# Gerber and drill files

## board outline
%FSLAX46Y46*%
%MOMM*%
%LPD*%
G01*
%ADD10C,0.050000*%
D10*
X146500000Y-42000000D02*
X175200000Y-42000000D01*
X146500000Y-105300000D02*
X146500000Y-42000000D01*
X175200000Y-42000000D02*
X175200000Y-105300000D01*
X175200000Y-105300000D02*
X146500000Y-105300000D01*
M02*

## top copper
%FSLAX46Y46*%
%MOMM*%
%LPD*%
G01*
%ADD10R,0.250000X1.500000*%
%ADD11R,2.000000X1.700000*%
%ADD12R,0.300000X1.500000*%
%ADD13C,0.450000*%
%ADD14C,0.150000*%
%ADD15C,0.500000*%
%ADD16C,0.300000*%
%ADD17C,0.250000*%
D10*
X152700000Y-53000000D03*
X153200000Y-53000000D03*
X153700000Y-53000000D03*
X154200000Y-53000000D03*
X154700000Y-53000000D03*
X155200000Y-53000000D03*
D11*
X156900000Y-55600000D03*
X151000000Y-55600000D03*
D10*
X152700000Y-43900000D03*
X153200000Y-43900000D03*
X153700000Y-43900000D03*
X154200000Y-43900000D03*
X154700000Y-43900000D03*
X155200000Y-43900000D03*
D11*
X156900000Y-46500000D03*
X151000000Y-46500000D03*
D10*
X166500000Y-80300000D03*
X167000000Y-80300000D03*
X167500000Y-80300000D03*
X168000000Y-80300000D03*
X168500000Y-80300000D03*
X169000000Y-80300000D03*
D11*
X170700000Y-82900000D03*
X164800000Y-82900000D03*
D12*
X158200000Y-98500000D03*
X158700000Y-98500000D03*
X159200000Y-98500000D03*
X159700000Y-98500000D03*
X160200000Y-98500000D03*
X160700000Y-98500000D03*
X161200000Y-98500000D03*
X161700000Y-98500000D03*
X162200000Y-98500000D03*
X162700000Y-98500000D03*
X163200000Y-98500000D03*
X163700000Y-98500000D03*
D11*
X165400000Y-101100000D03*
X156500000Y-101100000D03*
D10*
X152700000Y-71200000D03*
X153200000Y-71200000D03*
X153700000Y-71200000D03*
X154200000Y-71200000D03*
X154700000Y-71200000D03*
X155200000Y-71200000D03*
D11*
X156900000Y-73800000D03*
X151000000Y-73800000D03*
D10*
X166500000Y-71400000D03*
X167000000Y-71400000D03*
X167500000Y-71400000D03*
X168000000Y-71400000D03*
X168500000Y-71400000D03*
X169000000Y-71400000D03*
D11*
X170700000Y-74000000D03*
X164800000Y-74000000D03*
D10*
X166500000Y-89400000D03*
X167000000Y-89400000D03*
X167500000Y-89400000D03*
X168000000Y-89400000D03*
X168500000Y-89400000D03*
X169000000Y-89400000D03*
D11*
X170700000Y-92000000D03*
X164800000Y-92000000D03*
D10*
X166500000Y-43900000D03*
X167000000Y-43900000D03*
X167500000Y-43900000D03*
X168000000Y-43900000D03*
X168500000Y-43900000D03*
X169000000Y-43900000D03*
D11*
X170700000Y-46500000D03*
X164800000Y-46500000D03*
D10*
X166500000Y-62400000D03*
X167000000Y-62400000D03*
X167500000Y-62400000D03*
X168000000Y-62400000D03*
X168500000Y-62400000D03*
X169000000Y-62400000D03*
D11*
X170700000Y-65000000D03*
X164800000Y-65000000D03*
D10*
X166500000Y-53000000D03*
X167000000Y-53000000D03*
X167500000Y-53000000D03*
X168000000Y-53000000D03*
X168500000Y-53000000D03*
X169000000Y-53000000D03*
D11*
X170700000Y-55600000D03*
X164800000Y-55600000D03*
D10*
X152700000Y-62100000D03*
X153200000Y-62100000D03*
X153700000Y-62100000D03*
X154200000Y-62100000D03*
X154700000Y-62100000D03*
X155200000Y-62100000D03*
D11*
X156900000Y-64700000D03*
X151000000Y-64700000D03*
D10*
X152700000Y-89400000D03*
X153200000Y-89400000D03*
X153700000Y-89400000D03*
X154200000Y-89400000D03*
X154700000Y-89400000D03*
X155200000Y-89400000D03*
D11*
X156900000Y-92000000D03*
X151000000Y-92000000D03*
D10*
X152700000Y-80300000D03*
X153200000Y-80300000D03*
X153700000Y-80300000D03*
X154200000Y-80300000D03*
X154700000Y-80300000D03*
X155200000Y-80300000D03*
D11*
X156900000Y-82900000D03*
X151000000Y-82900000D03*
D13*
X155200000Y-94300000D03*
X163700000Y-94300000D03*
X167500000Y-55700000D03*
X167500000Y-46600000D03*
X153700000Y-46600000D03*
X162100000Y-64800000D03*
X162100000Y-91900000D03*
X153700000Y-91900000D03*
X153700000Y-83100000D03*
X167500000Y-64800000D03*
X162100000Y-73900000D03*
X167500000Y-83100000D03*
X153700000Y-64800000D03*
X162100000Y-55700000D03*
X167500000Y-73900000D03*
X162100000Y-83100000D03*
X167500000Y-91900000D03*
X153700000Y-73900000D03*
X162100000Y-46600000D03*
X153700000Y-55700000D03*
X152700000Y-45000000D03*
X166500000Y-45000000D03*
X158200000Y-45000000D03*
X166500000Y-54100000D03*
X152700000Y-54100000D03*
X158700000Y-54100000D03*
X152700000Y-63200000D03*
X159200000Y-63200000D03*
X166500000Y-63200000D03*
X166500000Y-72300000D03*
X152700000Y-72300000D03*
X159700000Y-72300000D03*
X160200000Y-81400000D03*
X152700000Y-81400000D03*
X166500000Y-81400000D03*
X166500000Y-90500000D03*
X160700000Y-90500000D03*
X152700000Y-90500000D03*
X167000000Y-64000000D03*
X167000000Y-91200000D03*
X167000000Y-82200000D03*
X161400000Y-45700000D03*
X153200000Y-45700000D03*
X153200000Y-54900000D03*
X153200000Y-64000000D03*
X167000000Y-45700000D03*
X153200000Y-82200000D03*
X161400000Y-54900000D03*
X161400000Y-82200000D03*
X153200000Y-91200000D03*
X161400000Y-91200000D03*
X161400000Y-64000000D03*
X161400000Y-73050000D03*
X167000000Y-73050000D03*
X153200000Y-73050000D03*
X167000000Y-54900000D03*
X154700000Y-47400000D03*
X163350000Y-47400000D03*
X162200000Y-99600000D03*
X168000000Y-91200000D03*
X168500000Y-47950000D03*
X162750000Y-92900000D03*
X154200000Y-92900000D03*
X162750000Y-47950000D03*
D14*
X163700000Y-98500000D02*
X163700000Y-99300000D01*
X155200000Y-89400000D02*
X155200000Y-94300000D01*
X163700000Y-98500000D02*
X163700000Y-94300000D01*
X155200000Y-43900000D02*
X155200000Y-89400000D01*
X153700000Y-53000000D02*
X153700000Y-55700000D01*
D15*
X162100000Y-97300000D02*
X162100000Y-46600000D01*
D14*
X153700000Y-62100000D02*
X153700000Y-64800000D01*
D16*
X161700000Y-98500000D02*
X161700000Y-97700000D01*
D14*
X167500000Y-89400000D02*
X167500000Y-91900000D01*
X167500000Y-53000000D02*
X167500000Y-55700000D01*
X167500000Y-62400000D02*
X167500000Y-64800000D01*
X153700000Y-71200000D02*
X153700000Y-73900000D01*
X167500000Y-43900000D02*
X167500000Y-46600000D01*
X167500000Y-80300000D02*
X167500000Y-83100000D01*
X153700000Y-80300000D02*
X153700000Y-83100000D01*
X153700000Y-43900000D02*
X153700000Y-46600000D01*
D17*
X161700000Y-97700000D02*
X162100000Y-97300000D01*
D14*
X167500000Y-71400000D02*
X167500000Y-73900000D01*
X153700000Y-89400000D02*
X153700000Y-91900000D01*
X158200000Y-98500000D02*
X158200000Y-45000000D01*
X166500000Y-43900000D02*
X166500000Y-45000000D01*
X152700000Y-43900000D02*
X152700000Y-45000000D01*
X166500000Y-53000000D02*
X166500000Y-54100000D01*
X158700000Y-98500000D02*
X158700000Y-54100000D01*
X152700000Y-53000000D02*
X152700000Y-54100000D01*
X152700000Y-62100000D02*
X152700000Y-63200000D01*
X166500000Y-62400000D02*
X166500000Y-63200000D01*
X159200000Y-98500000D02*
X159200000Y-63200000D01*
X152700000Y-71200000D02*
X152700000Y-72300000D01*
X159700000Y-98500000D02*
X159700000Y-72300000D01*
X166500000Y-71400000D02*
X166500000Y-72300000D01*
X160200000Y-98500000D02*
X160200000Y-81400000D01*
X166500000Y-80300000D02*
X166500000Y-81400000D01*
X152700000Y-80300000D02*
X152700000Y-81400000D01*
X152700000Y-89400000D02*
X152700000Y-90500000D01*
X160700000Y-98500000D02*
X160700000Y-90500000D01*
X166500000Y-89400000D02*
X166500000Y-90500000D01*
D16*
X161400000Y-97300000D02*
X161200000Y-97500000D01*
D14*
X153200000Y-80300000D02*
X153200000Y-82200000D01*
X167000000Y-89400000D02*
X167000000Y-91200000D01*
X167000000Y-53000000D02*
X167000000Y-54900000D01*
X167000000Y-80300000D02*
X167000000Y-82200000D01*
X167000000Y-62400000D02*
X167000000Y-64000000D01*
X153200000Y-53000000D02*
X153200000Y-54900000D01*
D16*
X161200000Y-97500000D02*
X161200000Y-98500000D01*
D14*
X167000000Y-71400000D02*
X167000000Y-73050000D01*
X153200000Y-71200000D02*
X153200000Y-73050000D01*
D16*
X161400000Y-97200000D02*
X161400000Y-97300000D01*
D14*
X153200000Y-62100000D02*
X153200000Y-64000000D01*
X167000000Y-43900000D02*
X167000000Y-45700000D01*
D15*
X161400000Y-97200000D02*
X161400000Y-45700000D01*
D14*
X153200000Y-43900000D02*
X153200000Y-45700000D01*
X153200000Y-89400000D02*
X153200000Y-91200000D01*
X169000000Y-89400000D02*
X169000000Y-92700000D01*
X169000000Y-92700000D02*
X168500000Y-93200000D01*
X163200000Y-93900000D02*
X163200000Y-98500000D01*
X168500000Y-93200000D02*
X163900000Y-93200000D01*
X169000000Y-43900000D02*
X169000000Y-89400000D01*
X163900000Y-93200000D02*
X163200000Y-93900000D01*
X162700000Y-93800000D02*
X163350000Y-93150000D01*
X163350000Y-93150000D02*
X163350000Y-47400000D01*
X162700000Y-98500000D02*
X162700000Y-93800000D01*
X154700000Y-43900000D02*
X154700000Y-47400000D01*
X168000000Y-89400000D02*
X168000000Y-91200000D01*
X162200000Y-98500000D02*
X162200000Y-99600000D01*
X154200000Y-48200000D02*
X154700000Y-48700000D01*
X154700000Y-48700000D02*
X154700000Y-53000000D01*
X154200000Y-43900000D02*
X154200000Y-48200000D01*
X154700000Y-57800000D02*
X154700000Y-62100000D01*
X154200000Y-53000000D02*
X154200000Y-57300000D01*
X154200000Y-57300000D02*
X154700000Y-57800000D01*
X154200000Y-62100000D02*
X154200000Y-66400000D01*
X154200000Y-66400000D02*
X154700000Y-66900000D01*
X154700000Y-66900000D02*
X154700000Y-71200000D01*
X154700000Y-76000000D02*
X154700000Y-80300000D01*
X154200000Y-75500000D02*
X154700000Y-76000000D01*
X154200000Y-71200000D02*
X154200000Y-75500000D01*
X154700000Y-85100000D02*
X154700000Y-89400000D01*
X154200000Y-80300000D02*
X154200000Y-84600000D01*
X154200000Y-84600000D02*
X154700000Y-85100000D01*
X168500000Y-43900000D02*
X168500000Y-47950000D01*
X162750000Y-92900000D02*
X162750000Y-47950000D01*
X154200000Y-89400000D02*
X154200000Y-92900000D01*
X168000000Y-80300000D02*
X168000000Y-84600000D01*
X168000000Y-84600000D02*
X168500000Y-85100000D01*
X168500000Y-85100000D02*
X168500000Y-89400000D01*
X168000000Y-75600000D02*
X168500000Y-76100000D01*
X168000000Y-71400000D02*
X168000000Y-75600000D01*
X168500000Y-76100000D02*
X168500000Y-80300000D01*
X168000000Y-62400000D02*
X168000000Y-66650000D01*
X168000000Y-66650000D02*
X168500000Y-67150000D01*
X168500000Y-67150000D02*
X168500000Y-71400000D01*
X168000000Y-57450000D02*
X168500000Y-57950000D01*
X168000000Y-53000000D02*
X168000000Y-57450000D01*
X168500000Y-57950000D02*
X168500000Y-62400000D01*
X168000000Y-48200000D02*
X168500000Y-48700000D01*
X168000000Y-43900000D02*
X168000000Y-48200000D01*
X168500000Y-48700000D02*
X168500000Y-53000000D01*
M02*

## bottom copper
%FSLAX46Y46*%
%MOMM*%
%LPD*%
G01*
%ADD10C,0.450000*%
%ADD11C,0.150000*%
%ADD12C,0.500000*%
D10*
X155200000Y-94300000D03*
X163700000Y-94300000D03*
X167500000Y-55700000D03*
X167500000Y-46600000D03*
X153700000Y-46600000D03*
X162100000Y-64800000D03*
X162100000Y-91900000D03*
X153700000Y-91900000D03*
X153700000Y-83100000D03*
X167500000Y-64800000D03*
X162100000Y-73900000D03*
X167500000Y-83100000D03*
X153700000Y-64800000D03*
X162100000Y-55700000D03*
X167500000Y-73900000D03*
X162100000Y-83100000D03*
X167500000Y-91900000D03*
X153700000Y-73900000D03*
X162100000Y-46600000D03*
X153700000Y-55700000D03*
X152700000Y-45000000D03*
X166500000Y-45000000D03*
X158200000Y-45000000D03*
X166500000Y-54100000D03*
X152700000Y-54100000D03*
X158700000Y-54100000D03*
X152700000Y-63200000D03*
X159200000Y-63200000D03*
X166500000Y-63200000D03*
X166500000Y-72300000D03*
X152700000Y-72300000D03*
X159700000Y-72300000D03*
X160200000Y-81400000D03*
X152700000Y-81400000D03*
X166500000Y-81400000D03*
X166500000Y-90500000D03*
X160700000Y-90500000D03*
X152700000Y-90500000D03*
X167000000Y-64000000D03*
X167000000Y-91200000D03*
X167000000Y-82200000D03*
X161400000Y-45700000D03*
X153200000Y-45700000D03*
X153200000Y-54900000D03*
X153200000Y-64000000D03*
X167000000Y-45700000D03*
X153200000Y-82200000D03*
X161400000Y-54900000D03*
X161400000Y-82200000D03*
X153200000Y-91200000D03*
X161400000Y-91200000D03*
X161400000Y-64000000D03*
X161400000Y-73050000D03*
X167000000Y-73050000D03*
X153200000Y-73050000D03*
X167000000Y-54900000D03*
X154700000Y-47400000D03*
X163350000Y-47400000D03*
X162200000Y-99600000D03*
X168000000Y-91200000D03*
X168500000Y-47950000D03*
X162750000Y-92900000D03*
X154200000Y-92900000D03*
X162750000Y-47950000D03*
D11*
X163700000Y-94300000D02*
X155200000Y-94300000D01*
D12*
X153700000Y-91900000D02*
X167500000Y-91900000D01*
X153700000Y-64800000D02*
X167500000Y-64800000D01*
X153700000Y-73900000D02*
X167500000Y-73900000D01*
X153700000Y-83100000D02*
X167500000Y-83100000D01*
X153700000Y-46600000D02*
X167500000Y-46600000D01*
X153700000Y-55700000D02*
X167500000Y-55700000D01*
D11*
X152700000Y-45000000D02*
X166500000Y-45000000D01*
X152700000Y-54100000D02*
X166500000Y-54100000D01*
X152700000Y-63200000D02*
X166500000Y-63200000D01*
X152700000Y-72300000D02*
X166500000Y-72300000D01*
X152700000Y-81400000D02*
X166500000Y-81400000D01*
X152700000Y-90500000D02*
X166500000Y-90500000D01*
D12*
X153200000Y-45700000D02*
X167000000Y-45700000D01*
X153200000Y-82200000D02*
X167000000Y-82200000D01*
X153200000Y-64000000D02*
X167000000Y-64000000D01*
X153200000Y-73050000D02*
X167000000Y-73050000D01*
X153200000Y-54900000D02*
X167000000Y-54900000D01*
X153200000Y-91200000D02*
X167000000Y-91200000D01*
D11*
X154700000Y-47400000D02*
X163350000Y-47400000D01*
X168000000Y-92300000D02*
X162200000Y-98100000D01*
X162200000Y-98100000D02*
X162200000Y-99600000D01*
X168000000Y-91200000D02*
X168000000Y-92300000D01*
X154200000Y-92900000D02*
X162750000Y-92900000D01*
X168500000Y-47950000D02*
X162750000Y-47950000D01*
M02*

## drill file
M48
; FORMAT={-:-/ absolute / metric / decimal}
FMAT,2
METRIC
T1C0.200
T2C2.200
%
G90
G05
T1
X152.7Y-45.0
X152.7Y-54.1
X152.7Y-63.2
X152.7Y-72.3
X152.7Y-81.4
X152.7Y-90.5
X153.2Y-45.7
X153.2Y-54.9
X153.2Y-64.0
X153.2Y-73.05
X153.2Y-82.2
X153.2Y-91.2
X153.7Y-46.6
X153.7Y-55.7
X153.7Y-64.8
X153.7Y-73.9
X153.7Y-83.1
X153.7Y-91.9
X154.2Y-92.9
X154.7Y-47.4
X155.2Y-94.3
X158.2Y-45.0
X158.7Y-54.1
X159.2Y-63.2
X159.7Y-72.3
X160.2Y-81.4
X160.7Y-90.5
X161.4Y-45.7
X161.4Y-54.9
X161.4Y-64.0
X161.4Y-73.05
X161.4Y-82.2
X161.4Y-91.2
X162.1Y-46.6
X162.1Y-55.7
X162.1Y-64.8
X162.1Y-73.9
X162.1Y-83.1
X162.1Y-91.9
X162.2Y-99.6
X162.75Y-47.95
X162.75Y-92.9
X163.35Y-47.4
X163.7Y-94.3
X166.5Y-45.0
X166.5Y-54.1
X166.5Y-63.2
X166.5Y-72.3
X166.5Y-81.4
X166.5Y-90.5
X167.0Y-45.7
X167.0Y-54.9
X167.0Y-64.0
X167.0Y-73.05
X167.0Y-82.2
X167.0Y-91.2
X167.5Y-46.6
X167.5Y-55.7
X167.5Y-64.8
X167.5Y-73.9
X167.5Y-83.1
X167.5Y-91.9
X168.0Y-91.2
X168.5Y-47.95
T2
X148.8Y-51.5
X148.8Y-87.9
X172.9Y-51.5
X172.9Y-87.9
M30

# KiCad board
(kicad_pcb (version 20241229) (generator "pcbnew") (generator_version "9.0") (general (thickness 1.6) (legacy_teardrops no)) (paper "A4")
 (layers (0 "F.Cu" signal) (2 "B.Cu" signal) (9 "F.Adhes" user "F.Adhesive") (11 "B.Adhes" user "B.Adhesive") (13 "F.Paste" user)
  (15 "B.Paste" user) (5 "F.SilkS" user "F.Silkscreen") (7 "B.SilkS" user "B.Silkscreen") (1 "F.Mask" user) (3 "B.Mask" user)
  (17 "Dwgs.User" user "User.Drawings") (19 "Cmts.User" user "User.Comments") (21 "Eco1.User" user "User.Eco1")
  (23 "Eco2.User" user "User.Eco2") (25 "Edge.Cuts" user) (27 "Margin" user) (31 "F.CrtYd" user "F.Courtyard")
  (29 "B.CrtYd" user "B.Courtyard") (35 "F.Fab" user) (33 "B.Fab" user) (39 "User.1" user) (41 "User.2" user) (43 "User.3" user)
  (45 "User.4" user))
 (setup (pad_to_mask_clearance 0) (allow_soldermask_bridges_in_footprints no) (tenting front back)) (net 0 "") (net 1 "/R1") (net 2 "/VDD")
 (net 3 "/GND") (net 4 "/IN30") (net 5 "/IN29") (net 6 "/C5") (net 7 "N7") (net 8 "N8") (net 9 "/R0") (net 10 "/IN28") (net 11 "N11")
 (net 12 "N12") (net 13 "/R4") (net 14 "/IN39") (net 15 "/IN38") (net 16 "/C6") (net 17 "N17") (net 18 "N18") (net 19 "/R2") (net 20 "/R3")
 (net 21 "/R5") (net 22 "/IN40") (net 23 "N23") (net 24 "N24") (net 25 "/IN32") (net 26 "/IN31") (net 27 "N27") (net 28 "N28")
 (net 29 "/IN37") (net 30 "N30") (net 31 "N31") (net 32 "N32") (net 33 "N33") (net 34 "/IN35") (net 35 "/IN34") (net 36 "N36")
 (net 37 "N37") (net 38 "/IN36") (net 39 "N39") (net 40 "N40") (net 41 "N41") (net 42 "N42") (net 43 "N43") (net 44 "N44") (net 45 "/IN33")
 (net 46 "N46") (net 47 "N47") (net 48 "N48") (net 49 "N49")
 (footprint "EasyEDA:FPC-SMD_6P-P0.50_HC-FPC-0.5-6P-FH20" (layer "F.Cu") (at 153.95 54.3)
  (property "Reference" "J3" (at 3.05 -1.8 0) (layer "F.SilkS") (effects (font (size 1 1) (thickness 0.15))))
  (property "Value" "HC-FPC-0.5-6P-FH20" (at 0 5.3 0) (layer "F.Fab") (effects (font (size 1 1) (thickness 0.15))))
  (pad "1" smd rect (at -1.25 -1.3) (size 0.25 1.5) (layers "F.Cu" "F.Mask" "F.Paste") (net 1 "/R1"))
  (pad "2" smd rect (at -0.75 -1.3) (size 0.25 1.5) (layers "F.Cu" "F.Mask" "F.Paste") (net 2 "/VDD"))
  (pad "3" smd rect (at -0.25 -1.3) (size 0.25 1.5) (layers "F.Cu" "F.Mask" "F.Paste") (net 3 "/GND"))
  (pad "4" smd rect (at 0.25 -1.3) (size 0.25 1.5) (layers "F.Cu" "F.Mask" "F.Paste") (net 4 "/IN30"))
  (pad "5" smd rect (at 0.75 -1.3) (size 0.25 1.5) (layers "F.Cu" "F.Mask" "F.Paste") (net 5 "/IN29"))
  (pad "6" smd rect (at 1.25 -1.3) (size 0.25 1.5) (layers "F.Cu" "F.Mask" "F.Paste") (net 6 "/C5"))
  (pad "7" smd rect (at 2.95 1.3) (size 2 1.7) (layers "F.Cu" "F.Mask" "F.Paste") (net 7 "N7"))
  (pad "8" smd rect (at -2.95 1.3) (size 2 1.7) (layers "F.Cu" "F.Mask" "F.Paste") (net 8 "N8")))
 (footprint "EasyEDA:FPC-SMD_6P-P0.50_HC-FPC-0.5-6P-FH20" (layer "F.Cu") (at 153.95 45.2)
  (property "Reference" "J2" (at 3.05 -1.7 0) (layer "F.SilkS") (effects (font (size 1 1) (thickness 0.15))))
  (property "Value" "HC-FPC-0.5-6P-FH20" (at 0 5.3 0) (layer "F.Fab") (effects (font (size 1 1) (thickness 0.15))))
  (pad "1" smd rect (at -1.25 -1.3) (size 0.25 1.5) (layers "F.Cu" "F.Mask" "F.Paste") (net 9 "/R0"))
  (pad "2" smd rect (at -0.75 -1.3) (size 0.25 1.5) (layers "F.Cu" "F.Mask" "F.Paste") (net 2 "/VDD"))
  (pad "3" smd rect (at -0.25 -1.3) (size 0.25 1.5) (layers "F.Cu" "F.Mask" "F.Paste") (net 3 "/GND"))
  (pad "4" smd rect (at 0.25 -1.3) (size 0.25 1.5) (layers "F.Cu" "F.Mask" "F.Paste") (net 5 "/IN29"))
  (pad "5" smd rect (at 0.75 -1.3) (size 0.25 1.5) (layers "F.Cu" "F.Mask" "F.Paste") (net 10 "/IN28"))
  (pad "6" smd rect (at 1.25 -1.3) (size 0.25 1.5) (layers "F.Cu" "F.Mask" "F.Paste") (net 6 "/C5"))
  (pad "7" smd rect (at 2.95 1.3) (size 2 1.7) (layers "F.Cu" "F.Mask" "F.Paste") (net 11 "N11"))
  (pad "8" smd rect (at -2.95 1.3) (size 2 1.7) (layers "F.Cu" "F.Mask" "F.Paste") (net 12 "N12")))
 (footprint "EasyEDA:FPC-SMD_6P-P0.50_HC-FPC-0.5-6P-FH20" (layer "F.Cu") (at 167.75 81.6)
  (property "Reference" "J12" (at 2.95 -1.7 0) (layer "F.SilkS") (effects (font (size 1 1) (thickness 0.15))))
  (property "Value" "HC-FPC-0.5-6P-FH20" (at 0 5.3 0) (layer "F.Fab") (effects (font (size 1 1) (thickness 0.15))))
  (pad "1" smd rect (at -1.25 -1.3) (size 0.25 1.5) (layers "F.Cu" "F.Mask" "F.Paste") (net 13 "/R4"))
  (pad "2" smd rect (at -0.75 -1.3) (size 0.25 1.5) (layers "F.Cu" "F.Mask" "F.Paste") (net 2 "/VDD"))
  (pad "3" smd rect (at -0.25 -1.3) (size 0.25 1.5) (layers "F.Cu" "F.Mask" "F.Paste") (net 3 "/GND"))
  (pad "4" smd rect (at 0.25 -1.3) (size 0.25 1.5) (layers "F.Cu" "F.Mask" "F.Paste") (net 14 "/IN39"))
  (pad "5" smd rect (at 0.75 -1.3) (size 0.25 1.5) (layers "F.Cu" "F.Mask" "F.Paste") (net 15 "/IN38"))
  (pad "6" smd rect (at 1.25 -1.3) (size 0.25 1.5) (layers "F.Cu" "F.Mask" "F.Paste") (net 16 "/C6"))
  (pad "7" smd rect (at 2.95 1.3) (size 2 1.7) (layers "F.Cu" "F.Mask" "F.Paste") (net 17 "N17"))
  (pad "8" smd rect (at -2.95 1.3) (size 2 1.7) (layers "F.Cu" "F.Mask" "F.Paste") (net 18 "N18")))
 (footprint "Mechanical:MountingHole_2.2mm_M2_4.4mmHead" (layer "F.Cu") (at 148.8 87.9)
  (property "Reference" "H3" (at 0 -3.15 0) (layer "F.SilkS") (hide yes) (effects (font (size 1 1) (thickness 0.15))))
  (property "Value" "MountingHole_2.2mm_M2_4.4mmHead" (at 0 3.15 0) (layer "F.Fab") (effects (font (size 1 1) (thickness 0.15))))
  (pad "" np_thru_hole circle (at 0 0) (size 2.2 2.2) (drill 2.2) (layers "*.Cu" "*.Mask")))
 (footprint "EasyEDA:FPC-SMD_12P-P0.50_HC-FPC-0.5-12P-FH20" (layer "F.Cu") (at 160.95 99.8)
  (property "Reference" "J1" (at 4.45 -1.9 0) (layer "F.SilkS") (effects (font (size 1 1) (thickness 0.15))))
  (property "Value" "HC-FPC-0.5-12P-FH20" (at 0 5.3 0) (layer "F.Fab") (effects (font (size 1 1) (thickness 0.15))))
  (pad "1" smd rect (at -2.75 -1.3) (size 0.3 1.5) (layers "F.Cu" "F.Mask" "F.Paste") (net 9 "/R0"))
  (pad "2" smd rect (at -2.25 -1.3) (size 0.3 1.5) (layers "F.Cu" "F.Mask" "F.Paste") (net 1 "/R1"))
  (pad "3" smd rect (at -1.75 -1.3) (size 0.3 1.5) (layers "F.Cu" "F.Mask" "F.Paste") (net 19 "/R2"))
  (pad "4" smd rect (at -1.25 -1.3) (size 0.3 1.5) (layers "F.Cu" "F.Mask" "F.Paste") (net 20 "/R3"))
  (pad "5" smd rect (at -0.75 -1.3) (size 0.3 1.5) (layers "F.Cu" "F.Mask" "F.Paste") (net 13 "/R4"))
  (pad "6" smd rect (at -0.25 -1.3) (size 0.3 1.5) (layers "F.Cu" "F.Mask" "F.Paste") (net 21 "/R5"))
  (pad "7" smd rect (at 0.25 -1.3) (size 0.3 1.5) (layers "F.Cu" "F.Mask" "F.Paste") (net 2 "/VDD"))
  (pad "8" smd rect (at 0.75 -1.3) (size 0.3 1.5) (layers "F.Cu" "F.Mask" "F.Paste") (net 3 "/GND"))
  (pad "9" smd rect (at 1.25 -1.3) (size 0.3 1.5) (layers "F.Cu" "F.Mask" "F.Paste") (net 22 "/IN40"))
  (pad "10" smd rect (at 1.75 -1.3) (size 0.3 1.5) (layers "F.Cu" "F.Mask" "F.Paste") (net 10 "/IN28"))
  (pad "11" smd rect (at 2.25 -1.3) (size 0.3 1.5) (layers "F.Cu" "F.Mask" "F.Paste") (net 16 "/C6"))
  (pad "12" smd rect (at 2.75 -1.3) (size 0.3 1.5) (layers "F.Cu" "F.Mask" "F.Paste") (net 6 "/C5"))
  (pad "13" smd rect (at 4.45 1.3) (size 2 1.7) (layers "F.Cu" "F.Mask" "F.Paste") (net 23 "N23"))
  (pad "14" smd rect (at -4.45 1.3) (size 2 1.7) (layers "F.Cu" "F.Mask" "F.Paste") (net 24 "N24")))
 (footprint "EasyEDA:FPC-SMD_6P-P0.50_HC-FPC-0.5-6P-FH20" (layer "F.Cu") (at 153.95 72.5)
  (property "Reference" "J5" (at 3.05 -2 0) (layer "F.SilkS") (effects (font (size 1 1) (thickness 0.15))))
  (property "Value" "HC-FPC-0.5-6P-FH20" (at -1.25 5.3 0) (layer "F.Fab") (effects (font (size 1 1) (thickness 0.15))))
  (pad "1" smd rect (at -1.25 -1.3) (size 0.25 1.5) (layers "F.Cu" "F.Mask" "F.Paste") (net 20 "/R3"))
  (pad "2" smd rect (at -0.75 -1.3) (size 0.25 1.5) (layers "F.Cu" "F.Mask" "F.Paste") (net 2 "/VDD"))
  (pad "3" smd rect (at -0.25 -1.3) (size 0.25 1.5) (layers "F.Cu" "F.Mask" "F.Paste") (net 3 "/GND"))
  (pad "4" smd rect (at 0.25 -1.3) (size 0.25 1.5) (layers "F.Cu" "F.Mask" "F.Paste") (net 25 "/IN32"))
  (pad "5" smd rect (at 0.75 -1.3) (size 0.25 1.5) (layers "F.Cu" "F.Mask" "F.Paste") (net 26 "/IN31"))
  (pad "6" smd rect (at 1.25 -1.3) (size 0.25 1.5) (layers "F.Cu" "F.Mask" "F.Paste") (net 6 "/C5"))
  (pad "7" smd rect (at 2.95 1.3) (size 2 1.7) (layers "F.Cu" "F.Mask" "F.Paste") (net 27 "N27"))
  (pad "8" smd rect (at -2.95 1.3) (size 2 1.7) (layers "F.Cu" "F.Mask" "F.Paste") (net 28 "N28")))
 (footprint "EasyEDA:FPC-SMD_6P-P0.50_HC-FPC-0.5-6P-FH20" (layer "F.Cu") (at 167.75 72.7)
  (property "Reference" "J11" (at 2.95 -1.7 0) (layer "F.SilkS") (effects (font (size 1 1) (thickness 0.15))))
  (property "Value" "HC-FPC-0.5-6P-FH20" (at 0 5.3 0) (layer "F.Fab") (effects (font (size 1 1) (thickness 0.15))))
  (pad "1" smd rect (at -1.25 -1.3) (size 0.25 1.5) (layers "F.Cu" "F.Mask" "F.Paste") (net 20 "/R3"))
  (pad "2" smd rect (at -0.75 -1.3) (size 0.25 1.5) (layers "F.Cu" "F.Mask" "F.Paste") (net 2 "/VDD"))
  (pad "3" smd rect (at -0.25 -1.3) (size 0.25 1.5) (layers "F.Cu" "F.Mask" "F.Paste") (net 3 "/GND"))
  (pad "4" smd rect (at 0.25 -1.3) (size 0.25 1.5) (layers "F.Cu" "F.Mask" "F.Paste") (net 15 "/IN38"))
  (pad "5" smd rect (at 0.75 -1.3) (size 0.25 1.5) (layers "F.Cu" "F.Mask" "F.Paste") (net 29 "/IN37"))
  (pad "6" smd rect (at 1.25 -1.3) (size 0.25 1.5) (layers "F.Cu" "F.Mask" "F.Paste") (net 16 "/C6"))
  (pad "7" smd rect (at 2.95 1.3) (size 2 1.7) (layers "F.Cu" "F.Mask" "F.Paste") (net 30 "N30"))
  (pad "8" smd rect (at -2.95 1.3) (size 2 1.7) (layers "F.Cu" "F.Mask" "F.Paste") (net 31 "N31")))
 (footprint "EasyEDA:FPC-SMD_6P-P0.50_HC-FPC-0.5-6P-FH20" (layer "F.Cu") (at 167.75 90.7)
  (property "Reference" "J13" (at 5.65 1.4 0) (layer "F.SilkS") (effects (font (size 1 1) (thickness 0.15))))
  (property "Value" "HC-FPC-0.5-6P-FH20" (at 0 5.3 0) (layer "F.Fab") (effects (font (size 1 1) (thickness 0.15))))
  (pad "1" smd rect (at -1.25 -1.3) (size 0.25 1.5) (layers "F.Cu" "F.Mask" "F.Paste") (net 21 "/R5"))
  (pad "2" smd rect (at -0.75 -1.3) (size 0.25 1.5) (layers "F.Cu" "F.Mask" "F.Paste") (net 2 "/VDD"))
  (pad "3" smd rect (at -0.25 -1.3) (size 0.25 1.5) (layers "F.Cu" "F.Mask" "F.Paste") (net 3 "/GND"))
  (pad "4" smd rect (at 0.25 -1.3) (size 0.25 1.5) (layers "F.Cu" "F.Mask" "F.Paste") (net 22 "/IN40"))
  (pad "5" smd rect (at 0.75 -1.3) (size 0.25 1.5) (layers "F.Cu" "F.Mask" "F.Paste") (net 14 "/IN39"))
  (pad "6" smd rect (at 1.25 -1.3) (size 0.25 1.5) (layers "F.Cu" "F.Mask" "F.Paste") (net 16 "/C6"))
  (pad "7" smd rect (at 2.95 1.3) (size 2 1.7) (layers "F.Cu" "F.Mask" "F.Paste") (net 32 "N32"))
  (pad "8" smd rect (at -2.95 1.3) (size 2 1.7) (layers "F.Cu" "F.Mask" "F.Paste") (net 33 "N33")))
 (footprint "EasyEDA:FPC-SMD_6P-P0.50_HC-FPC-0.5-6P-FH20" (layer "F.Cu") (at 167.75 45.2)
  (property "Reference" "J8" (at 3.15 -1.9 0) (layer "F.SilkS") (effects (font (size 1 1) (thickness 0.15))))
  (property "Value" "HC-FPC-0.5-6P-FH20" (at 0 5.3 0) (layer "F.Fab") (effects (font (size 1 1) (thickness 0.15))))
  (pad "1" smd rect (at -1.25 -1.3) (size 0.25 1.5) (layers "F.Cu" "F.Mask" "F.Paste") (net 9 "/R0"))
  (pad "2" smd rect (at -0.75 -1.3) (size 0.25 1.5) (layers "F.Cu" "F.Mask" "F.Paste") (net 2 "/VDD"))
  (pad "3" smd rect (at -0.25 -1.3) (size 0.25 1.5) (layers "F.Cu" "F.Mask" "F.Paste") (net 3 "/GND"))
  (pad "4" smd rect (at 0.25 -1.3) (size 0.25 1.5) (layers "F.Cu" "F.Mask" "F.Paste") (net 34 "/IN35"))
  (pad "5" smd rect (at 0.75 -1.3) (size 0.25 1.5) (layers "F.Cu" "F.Mask" "F.Paste") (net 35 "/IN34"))
  (pad "6" smd rect (at 1.25 -1.3) (size 0.25 1.5) (layers "F.Cu" "F.Mask" "F.Paste") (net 16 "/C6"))
  (pad "7" smd rect (at 2.95 1.3) (size 2 1.7) (layers "F.Cu" "F.Mask" "F.Paste") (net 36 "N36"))
  (pad "8" smd rect (at -2.95 1.3) (size 2 1.7) (layers "F.Cu" "F.Mask" "F.Paste") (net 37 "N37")))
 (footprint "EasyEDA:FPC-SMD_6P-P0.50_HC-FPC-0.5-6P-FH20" (layer "F.Cu") (at 167.75 63.7)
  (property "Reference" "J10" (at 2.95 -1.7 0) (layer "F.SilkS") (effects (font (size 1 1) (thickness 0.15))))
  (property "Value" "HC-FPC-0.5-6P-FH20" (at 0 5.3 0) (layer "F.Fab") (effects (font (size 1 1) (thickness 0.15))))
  (pad "1" smd rect (at -1.25 -1.3) (size 0.25 1.5) (layers "F.Cu" "F.Mask" "F.Paste") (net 19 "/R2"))
  (pad "2" smd rect (at -0.75 -1.3) (size 0.25 1.5) (layers "F.Cu" "F.Mask" "F.Paste") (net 2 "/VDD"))
  (pad "3" smd rect (at -0.25 -1.3) (size 0.25 1.5) (layers "F.Cu" "F.Mask" "F.Paste") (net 3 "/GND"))
  (pad "4" smd rect (at 0.25 -1.3) (size 0.25 1.5) (layers "F.Cu" "F.Mask" "F.Paste") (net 29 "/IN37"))
  (pad "5" smd rect (at 0.75 -1.3) (size 0.25 1.5) (layers "F.Cu" "F.Mask" "F.Paste") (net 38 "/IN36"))
  (pad "6" smd rect (at 1.25 -1.3) (size 0.25 1.5) (layers "F.Cu" "F.Mask" "F.Paste") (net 16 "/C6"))
  (pad "7" smd rect (at 2.95 1.3) (size 2 1.7) (layers "F.Cu" "F.Mask" "F.Paste") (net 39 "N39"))
  (pad "8" smd rect (at -2.95 1.3) (size 2 1.7) (layers "F.Cu" "F.Mask" "F.Paste") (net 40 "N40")))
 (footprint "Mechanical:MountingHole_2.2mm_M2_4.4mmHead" (layer "F.Cu") (at 172.9 51.5)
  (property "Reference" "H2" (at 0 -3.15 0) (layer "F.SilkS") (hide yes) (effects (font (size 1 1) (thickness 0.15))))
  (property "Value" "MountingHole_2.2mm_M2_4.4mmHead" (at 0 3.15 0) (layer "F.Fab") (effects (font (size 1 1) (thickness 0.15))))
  (pad "" np_thru_hole circle (at 0 0) (size 2.2 2.2) (drill 2.2) (layers "*.Cu" "*.Mask")))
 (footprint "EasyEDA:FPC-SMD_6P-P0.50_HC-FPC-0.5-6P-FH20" (layer "F.Cu") (at 167.75 54.3)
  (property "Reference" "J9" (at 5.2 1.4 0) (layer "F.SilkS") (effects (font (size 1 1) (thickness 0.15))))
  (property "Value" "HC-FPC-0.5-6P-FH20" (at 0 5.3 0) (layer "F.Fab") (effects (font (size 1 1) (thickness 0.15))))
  (pad "1" smd rect (at -1.25 -1.3) (size 0.25 1.5) (layers "F.Cu" "F.Mask" "F.Paste") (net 1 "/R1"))
  (pad "2" smd rect (at -0.75 -1.3) (size 0.25 1.5) (layers "F.Cu" "F.Mask" "F.Paste") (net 2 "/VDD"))
  (pad "3" smd rect (at -0.25 -1.3) (size 0.25 1.5) (layers "F.Cu" "F.Mask" "F.Paste") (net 3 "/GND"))
  (pad "4" smd rect (at 0.25 -1.3) (size 0.25 1.5) (layers "F.Cu" "F.Mask" "F.Paste") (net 38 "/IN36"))
  (pad "5" smd rect (at 0.75 -1.3) (size 0.25 1.5) (layers "F.Cu" "F.Mask" "F.Paste") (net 34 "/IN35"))
  (pad "6" smd rect (at 1.25 -1.3) (size 0.25 1.5) (layers "F.Cu" "F.Mask" "F.Paste") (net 16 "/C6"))
  (pad "7" smd rect (at 2.95 1.3) (size 2 1.7) (layers "F.Cu" "F.Mask" "F.Paste") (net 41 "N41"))
  (pad "8" smd rect (at -2.95 1.3) (size 2 1.7) (layers "F.Cu" "F.Mask" "F.Paste") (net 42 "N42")))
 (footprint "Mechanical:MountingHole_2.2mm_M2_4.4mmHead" (layer "F.Cu") (at 148.8 51.5)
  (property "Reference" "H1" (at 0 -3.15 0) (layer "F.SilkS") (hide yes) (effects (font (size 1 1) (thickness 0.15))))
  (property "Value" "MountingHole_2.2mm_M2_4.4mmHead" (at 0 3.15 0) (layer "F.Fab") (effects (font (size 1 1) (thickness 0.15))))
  (pad "" np_thru_hole circle (at 0 0) (size 2.2 2.2) (drill 2.2) (layers "*.Cu" "*.Mask")))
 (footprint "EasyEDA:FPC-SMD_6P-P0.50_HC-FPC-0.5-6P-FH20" (layer "F.Cu") (at 153.95 63.4)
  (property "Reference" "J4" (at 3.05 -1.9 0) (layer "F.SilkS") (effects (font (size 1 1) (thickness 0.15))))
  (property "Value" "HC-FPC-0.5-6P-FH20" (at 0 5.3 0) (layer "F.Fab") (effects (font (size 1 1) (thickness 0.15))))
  (pad "1" smd rect (at -1.25 -1.3) (size 0.25 1.5) (layers "F.Cu" "F.Mask" "F.Paste") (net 19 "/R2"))
  (pad "2" smd rect (at -0.75 -1.3) (size 0.25 1.5) (layers "F.Cu" "F.Mask" "F.Paste") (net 2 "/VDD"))
  (pad "3" smd rect (at -0.25 -1.3) (size 0.25 1.5) (layers "F.Cu" "F.Mask" "F.Paste") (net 3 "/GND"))
  (pad "4" smd rect (at 0.25 -1.3) (size 0.25 1.5) (layers "F.Cu" "F.Mask" "F.Paste") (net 26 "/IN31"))
  (pad "5" smd rect (at 0.75 -1.3) (size 0.25 1.5) (layers "F.Cu" "F.Mask" "F.Paste") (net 4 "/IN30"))
  (pad "6" smd rect (at 1.25 -1.3) (size 0.25 1.5) (layers "F.Cu" "F.Mask" "F.Paste") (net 6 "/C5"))
  (pad "7" smd rect (at 2.95 1.3) (size 2 1.7) (layers "F.Cu" "F.Mask" "F.Paste") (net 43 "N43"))
  (pad "8" smd rect (at -2.95 1.3) (size 2 1.7) (layers "F.Cu" "F.Mask" "F.Paste") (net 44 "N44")))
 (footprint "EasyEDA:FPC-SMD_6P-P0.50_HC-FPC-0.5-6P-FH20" (layer "F.Cu") (at 153.95 90.7)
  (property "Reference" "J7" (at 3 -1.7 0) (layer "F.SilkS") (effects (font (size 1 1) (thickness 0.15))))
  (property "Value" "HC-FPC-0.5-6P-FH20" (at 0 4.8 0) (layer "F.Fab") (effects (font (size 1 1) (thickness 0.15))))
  (pad "1" smd rect (at -1.25 -1.3) (size 0.25 1.5) (layers "F.Cu" "F.Mask" "F.Paste") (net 21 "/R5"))
  (pad "2" smd rect (at -0.75 -1.3) (size 0.25 1.5) (layers "F.Cu" "F.Mask" "F.Paste") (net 2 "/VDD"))
  (pad "3" smd rect (at -0.25 -1.3) (size 0.25 1.5) (layers "F.Cu" "F.Mask" "F.Paste") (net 3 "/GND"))
  (pad "4" smd rect (at 0.25 -1.3) (size 0.25 1.5) (layers "F.Cu" "F.Mask" "F.Paste") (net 35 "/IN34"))
  (pad "5" smd rect (at 0.75 -1.3) (size 0.25 1.5) (layers "F.Cu" "F.Mask" "F.Paste") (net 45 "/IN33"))
  (pad "6" smd rect (at 1.25 -1.3) (size 0.25 1.5) (layers "F.Cu" "F.Mask" "F.Paste") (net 6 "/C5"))
  (pad "7" smd rect (at 2.95 1.3) (size 2 1.7) (layers "F.Cu" "F.Mask" "F.Paste") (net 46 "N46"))
  (pad "8" smd rect (at -2.95 1.3) (size 2 1.7) (layers "F.Cu" "F.Mask" "F.Paste") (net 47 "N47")))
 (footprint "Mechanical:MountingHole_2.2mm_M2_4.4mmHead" (layer "F.Cu") (at 172.9 87.9)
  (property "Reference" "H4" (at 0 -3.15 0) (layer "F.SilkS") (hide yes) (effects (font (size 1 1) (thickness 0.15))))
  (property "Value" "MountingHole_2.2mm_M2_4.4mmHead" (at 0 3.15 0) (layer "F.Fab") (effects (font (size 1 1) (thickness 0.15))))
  (pad "" np_thru_hole circle (at 0 0) (size 2.2 2.2) (drill 2.2) (layers "*.Cu" "*.Mask")))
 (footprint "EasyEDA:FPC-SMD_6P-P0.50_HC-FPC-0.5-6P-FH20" (layer "F.Cu") (at 153.95 81.6)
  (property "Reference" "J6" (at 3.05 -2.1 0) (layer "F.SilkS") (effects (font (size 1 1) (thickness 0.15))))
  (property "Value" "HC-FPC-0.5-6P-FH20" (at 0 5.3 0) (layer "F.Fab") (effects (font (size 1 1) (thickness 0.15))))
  (pad "1" smd rect (at -1.25 -1.3) (size 0.25 1.5) (layers "F.Cu" "F.Mask" "F.Paste") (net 13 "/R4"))
  (pad "2" smd rect (at -0.75 -1.3) (size 0.25 1.5) (layers "F.Cu" "F.Mask" "F.Paste") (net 2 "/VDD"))
  (pad "3" smd rect (at -0.25 -1.3) (size 0.25 1.5) (layers "F.Cu" "F.Mask" "F.Paste") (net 3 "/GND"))
  (pad "4" smd rect (at 0.25 -1.3) (size 0.25 1.5) (layers "F.Cu" "F.Mask" "F.Paste") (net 45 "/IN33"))
  (pad "5" smd rect (at 0.75 -1.3) (size 0.25 1.5) (layers "F.Cu" "F.Mask" "F.Paste") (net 25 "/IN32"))
  (pad "6" smd rect (at 1.25 -1.3) (size 0.25 1.5) (layers "F.Cu" "F.Mask" "F.Paste") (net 6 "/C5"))
  (pad "7" smd rect (at 2.95 1.3) (size 2 1.7) (layers "F.Cu" "F.Mask" "F.Paste") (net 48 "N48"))
  (pad "8" smd rect (at -2.95 1.3) (size 2 1.7) (layers "F.Cu" "F.Mask" "F.Paste") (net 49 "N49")))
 (gr_line (start 146.5 42) (end 175.2 42) (stroke (width 0.05) (type default)) (layer "Edge.Cuts"))
 (gr_line (start 146.5 105.3) (end 146.5 42) (stroke (width 0.05) (type default)) (layer "Edge.Cuts"))
 (gr_line (start 175.2 42) (end 175.2 105.3) (stroke (width 0.05) (type default)) (layer "Edge.Cuts"))
 (gr_line (start 175.2 105.3) (end 146.5 105.3) (stroke (width 0.05) (type default)) (layer "Edge.Cuts"))
 (segment (start 163.7 98.5) (end 163.7 99.3) (width 0.15) (layer "F.Cu") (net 6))
 (segment (start 155.2 89.4) (end 155.2 94.3) (width 0.15) (layer "F.Cu") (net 6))
 (segment (start 163.7 98.5) (end 163.7 94.3) (width 0.15) (layer "F.Cu") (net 6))
 (segment (start 155.2 43.9) (end 155.2 89.4) (width 0.15) (layer "F.Cu") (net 6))
 (via (at 155.2 94.3) (size 0.45) (drill 0.2) (layers "F.Cu" "B.Cu") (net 6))
 (via (at 163.7 94.3) (size 0.45) (drill 0.2) (layers "F.Cu" "B.Cu") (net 6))
 (segment (start 163.7 94.3) (end 155.2 94.3) (width 0.15) (layer "B.Cu") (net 6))
 (segment (start 153.7 53) (end 153.7 55.7) (width 0.15) (layer "F.Cu") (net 3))
 (segment (start 162.1 97.3) (end 162.1 46.6) (width 0.5) (layer "F.Cu") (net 3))
 (segment (start 153.7 62.1) (end 153.7 64.8) (width 0.15) (layer "F.Cu") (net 3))
 (segment (start 161.7 98.5) (end 161.7 97.7) (width 0.3) (layer "F.Cu") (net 3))
 (segment (start 167.5 89.4) (end 167.5 91.9) (width 0.15) (layer "F.Cu") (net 3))
 (segment (start 167.5 53) (end 167.5 55.7) (width 0.15) (layer "F.Cu") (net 3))
 (segment (start 167.5 62.4) (end 167.5 64.8) (width 0.15) (layer "F.Cu") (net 3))
 (segment (start 153.7 71.2) (end 153.7 73.9) (width 0.15) (layer "F.Cu") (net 3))
 (segment (start 167.5 43.9) (end 167.5 46.6) (width 0.15) (layer "F.Cu") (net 3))
 (segment (start 167.5 80.3) (end 167.5 83.1) (width 0.15) (layer "F.Cu") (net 3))
 (segment (start 153.7 80.3) (end 153.7 83.1) (width 0.15) (layer "F.Cu") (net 3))
 (segment (start 153.7 43.9) (end 153.7 46.6) (width 0.15) (layer "F.Cu") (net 3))
 (segment (start 161.7 97.7) (end 162.1 97.3) (width 0.25) (layer "F.Cu") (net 3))
 (segment (start 167.5 71.4) (end 167.5 73.9) (width 0.15) (layer "F.Cu") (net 3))
 (segment (start 153.7 89.4) (end 153.7 91.9) (width 0.15) (layer "F.Cu") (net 3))
 (via (at 167.5 55.7) (size 0.45) (drill 0.2) (layers "F.Cu" "B.Cu") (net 3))
 (via (at 167.5 46.6) (size 0.45) (drill 0.2) (layers "F.Cu" "B.Cu") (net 3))
 (via (at 153.7 46.6) (size 0.45) (drill 0.2) (layers "F.Cu" "B.Cu") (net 3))
 (via (at 162.1 64.8) (size 0.45) (drill 0.2) (layers "F.Cu" "B.Cu") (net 3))
 (via (at 162.1 91.9) (size 0.45) (drill 0.2) (layers "F.Cu" "B.Cu") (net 3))
 (via (at 153.7 91.9) (size 0.45) (drill 0.2) (layers "F.Cu" "B.Cu") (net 3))
 (via (at 153.7 83.1) (size 0.45) (drill 0.2) (layers "F.Cu" "B.Cu") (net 3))
 (via (at 167.5 64.8) (size 0.45) (drill 0.2) (layers "F.Cu" "B.Cu") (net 3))
 (via (at 162.1 73.9) (size 0.45) (drill 0.2) (layers "F.Cu" "B.Cu") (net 3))
 (via (at 167.5 83.1) (size 0.45) (drill 0.2) (layers "F.Cu" "B.Cu") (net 3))
 (via (at 153.7 64.8) (size 0.45) (drill 0.2) (layers "F.Cu" "B.Cu") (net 3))
 (via (at 162.1 55.7) (size 0.45) (drill 0.2) (layers "F.Cu" "B.Cu") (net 3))
 (via (at 167.5 73.9) (size 0.45) (drill 0.2) (layers "F.Cu" "B.Cu") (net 3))
 (via (at 162.1 83.1) (size 0.45) (drill 0.2) (layers "F.Cu" "B.Cu") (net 3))
 (via (at 167.5 91.9) (size 0.45) (drill 0.2) (layers "F.Cu" "B.Cu") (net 3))
 (via (at 153.7 73.9) (size 0.45) (drill 0.2) (layers "F.Cu" "B.Cu") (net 3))
 (via (at 162.1 46.6) (size 0.45) (drill 0.2) (layers "F.Cu" "B.Cu") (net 3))
 (via (at 153.7 55.7) (size 0.45) (drill 0.2) (layers "F.Cu" "B.Cu") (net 3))
 (segment (start 153.7 91.9) (end 167.5 91.9) (width 0.5) (layer "B.Cu") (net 3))
 (segment (start 153.7 64.8) (end 167.5 64.8) (width 0.5) (layer "B.Cu") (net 3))
 (segment (start 153.7 73.9) (end 167.5 73.9) (width 0.5) (layer "B.Cu") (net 3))
 (segment (start 153.7 83.1) (end 167.5 83.1) (width 0.5) (layer "B.Cu") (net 3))
 (segment (start 153.7 46.6) (end 167.5 46.6) (width 0.5) (layer "B.Cu") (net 3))
 (segment (start 153.7 55.7) (end 167.5 55.7) (width 0.5) (layer "B.Cu") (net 3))
 (segment (start 158.2 98.5) (end 158.2 45) (width 0.15) (layer "F.Cu") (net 9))
 (segment (start 166.5 43.9) (end 166.5 45) (width 0.15) (layer "F.Cu") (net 9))
 (segment (start 152.7 43.9) (end 152.7 45) (width 0.15) (layer "F.Cu") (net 9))
 (via (at 152.7 45) (size 0.45) (drill 0.2) (layers "F.Cu" "B.Cu") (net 9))
 (via (at 166.5 45) (size 0.45) (drill 0.2) (layers "F.Cu" "B.Cu") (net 9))
 (via (at 158.2 45) (size 0.45) (drill 0.2) (layers "F.Cu" "B.Cu") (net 9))
 (segment (start 152.7 45) (end 166.5 45) (width 0.15) (layer "B.Cu") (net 9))
 (segment (start 166.5 53) (end 166.5 54.1) (width 0.15) (layer "F.Cu") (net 1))
 (segment (start 158.7 98.5) (end 158.7 54.1) (width 0.15) (layer "F.Cu") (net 1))
 (segment (start 152.7 53) (end 152.7 54.1) (width 0.15) (layer "F.Cu") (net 1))
 (via (at 166.5 54.1) (size 0.45) (drill 0.2) (layers "F.Cu" "B.Cu") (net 1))
 (via (at 152.7 54.1) (size 0.45) (drill 0.2) (layers "F.Cu" "B.Cu") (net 1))
 (via (at 158.7 54.1) (size 0.45) (drill 0.2) (layers "F.Cu" "B.Cu") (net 1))
 (segment (start 152.7 54.1) (end 166.5 54.1) (width 0.15) (layer "B.Cu") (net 1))
 (segment (start 152.7 62.1) (end 152.7 63.2) (width 0.15) (layer "F.Cu") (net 19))
 (segment (start 166.5 62.4) (end 166.5 63.2) (width 0.15) (layer "F.Cu") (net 19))
 (segment (start 159.2 98.5) (end 159.2 63.2) (width 0.15) (layer "F.Cu") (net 19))
 (via (at 152.7 63.2) (size 0.45) (drill 0.2) (layers "F.Cu" "B.Cu") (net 19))
 (via (at 159.2 63.2) (size 0.45) (drill 0.2) (layers "F.Cu" "B.Cu") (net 19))
 (via (at 166.5 63.2) (size 0.45) (drill 0.2) (layers "F.Cu" "B.Cu") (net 19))
 (segment (start 152.7 63.2) (end 166.5 63.2) (width 0.15) (layer "B.Cu") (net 19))
 (segment (start 152.7 71.2) (end 152.7 72.3) (width 0.15) (layer "F.Cu") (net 20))
 (segment (start 159.7 98.5) (end 159.7 72.3) (width 0.15) (layer "F.Cu") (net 20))
 (segment (start 166.5 71.4) (end 166.5 72.3) (width 0.15) (layer "F.Cu") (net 20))
 (via (at 166.5 72.3) (size 0.45) (drill 0.2) (layers "F.Cu" "B.Cu") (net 20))
 (via (at 152.7 72.3) (size 0.45) (drill 0.2) (layers "F.Cu" "B.Cu") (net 20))
 (via (at 159.7 72.3) (size 0.45) (drill 0.2) (layers "F.Cu" "B.Cu") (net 20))
 (segment (start 152.7 72.3) (end 166.5 72.3) (width 0.15) (layer "B.Cu") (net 20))
 (segment (start 160.2 98.5) (end 160.2 81.4) (width 0.15) (layer "F.Cu") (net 13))
 (segment (start 166.5 80.3) (end 166.5 81.4) (width 0.15) (layer "F.Cu") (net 13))
 (segment (start 152.7 80.3) (end 152.7 81.4) (width 0.15) (layer "F.Cu") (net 13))
 (via (at 160.2 81.4) (size 0.45) (drill 0.2) (layers "F.Cu" "B.Cu") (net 13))
 (via (at 152.7 81.4) (size 0.45) (drill 0.2) (layers "F.Cu" "B.Cu") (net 13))
 (via (at 166.5 81.4) (size 0.45) (drill 0.2) (layers "F.Cu" "B.Cu") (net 13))
 (segment (start 152.7 81.4) (end 166.5 81.4) (width 0.15) (layer "B.Cu") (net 13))
 (segment (start 152.7 89.4) (end 152.7 90.5) (width 0.15) (layer "F.Cu") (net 21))
 (segment (start 160.7 98.5) (end 160.7 90.5) (width 0.15) (layer "F.Cu") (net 21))
 (segment (start 166.5 89.4) (end 166.5 90.5) (width 0.15) (layer "F.Cu") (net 21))
 (via (at 166.5 90.5) (size 0.45) (drill 0.2) (layers "F.Cu" "B.Cu") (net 21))
 (via (at 160.7 90.5) (size 0.45) (drill 0.2) (layers "F.Cu" "B.Cu") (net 21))
 (via (at 152.7 90.5) (size 0.45) (drill 0.2) (layers "F.Cu" "B.Cu") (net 21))
 (segment (start 152.7 90.5) (end 166.5 90.5) (width 0.15) (layer "B.Cu") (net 21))
 (segment (start 161.4 97.3) (end 161.2 97.5) (width 0.3) (layer "F.Cu") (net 2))
 (segment (start 153.2 80.3) (end 153.2 82.2) (width 0.15) (layer "F.Cu") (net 2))
 (segment (start 167 89.4) (end 167 91.2) (width 0.15) (layer "F.Cu") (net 2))
 (segment (start 167 53) (end 167 54.9) (width 0.15) (layer "F.Cu") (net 2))
 (segment (start 167 80.3) (end 167 82.2) (width 0.15) (layer "F.Cu") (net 2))
 (segment (start 167 62.4) (end 167 64) (width 0.15) (layer "F.Cu") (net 2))
 (segment (start 153.2 53) (end 153.2 54.9) (width 0.15) (layer "F.Cu") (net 2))
 (segment (start 161.2 97.5) (end 161.2 98.5) (width 0.3) (layer "F.Cu") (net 2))
 (segment (start 167 71.4) (end 167 73.05) (width 0.15) (layer "F.Cu") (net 2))
 (segment (start 153.2 71.2) (end 153.2 73.05) (width 0.15) (layer "F.Cu") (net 2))
 (segment (start 161.4 97.2) (end 161.4 97.3) (width 0.3) (layer "F.Cu") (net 2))
 (segment (start 153.2 62.1) (end 153.2 64) (width 0.15) (layer "F.Cu") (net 2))
 (segment (start 167 43.9) (end 167 45.7) (width 0.15) (layer "F.Cu") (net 2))
 (segment (start 161.4 97.2) (end 161.4 45.7) (width 0.5) (layer "F.Cu") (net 2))
 (segment (start 153.2 43.9) (end 153.2 45.7) (width 0.15) (layer "F.Cu") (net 2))
 (segment (start 153.2 89.4) (end 153.2 91.2) (width 0.15) (layer "F.Cu") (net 2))
 (via (at 167 64) (size 0.45) (drill 0.2) (layers "F.Cu" "B.Cu") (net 2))
 (via (at 167 91.2) (size 0.45) (drill 0.2) (layers "F.Cu" "B.Cu") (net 2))
 (via (at 167 82.2) (size 0.45) (drill 0.2) (layers "F.Cu" "B.Cu") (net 2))
 (via (at 161.4 45.7) (size 0.45) (drill 0.2) (layers "F.Cu" "B.Cu") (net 2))
 (via (at 153.2 45.7) (size 0.45) (drill 0.2) (layers "F.Cu" "B.Cu") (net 2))
 (via (at 153.2 54.9) (size 0.45) (drill 0.2) (layers "F.Cu" "B.Cu") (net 2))
 (via (at 153.2 64) (size 0.45) (drill 0.2) (layers "F.Cu" "B.Cu") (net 2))
 (via (at 167 45.7) (size 0.45) (drill 0.2) (layers "F.Cu" "B.Cu") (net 2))
 (via (at 153.2 82.2) (size 0.45) (drill 0.2) (layers "F.Cu" "B.Cu") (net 2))
 (via (at 161.4 54.9) (size 0.45) (drill 0.2) (layers "F.Cu" "B.Cu") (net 2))
 (via (at 161.4 82.2) (size 0.45) (drill 0.2) (layers "F.Cu" "B.Cu") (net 2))
 (via (at 153.2 91.2) (size 0.45) (drill 0.2) (layers "F.Cu" "B.Cu") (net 2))
 (via (at 161.4 91.2) (size 0.45) (drill 0.2) (layers "F.Cu" "B.Cu") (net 2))
 (via (at 161.4 64) (size 0.45) (drill 0.2) (layers "F.Cu" "B.Cu") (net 2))
 (via (at 161.4 73.05) (size 0.45) (drill 0.2) (layers "F.Cu" "B.Cu") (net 2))
 (via (at 167 73.05) (size 0.45) (drill 0.2) (layers "F.Cu" "B.Cu") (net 2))
 (via (at 153.2 73.05) (size 0.45) (drill 0.2) (layers "F.Cu" "B.Cu") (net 2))
 (via (at 167 54.9) (size 0.45) (drill 0.2) (layers "F.Cu" "B.Cu") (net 2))
 (segment (start 153.2 45.7) (end 167 45.7) (width 0.5) (layer "B.Cu") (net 2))
 (segment (start 153.2 82.2) (end 167 82.2) (width 0.5) (layer "B.Cu") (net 2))
 (segment (start 153.2 64) (end 167 64) (width 0.5) (layer "B.Cu") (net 2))
 (segment (start 153.2 73.05) (end 167 73.05) (width 0.5) (layer "B.Cu") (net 2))
 (segment (start 153.2 54.9) (end 167 54.9) (width 0.5) (layer "B.Cu") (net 2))
 (segment (start 153.2 91.2) (end 167 91.2) (width 0.5) (layer "B.Cu") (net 2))
 (segment (start 169 89.4) (end 169 92.7) (width 0.15) (layer "F.Cu") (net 16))
 (segment (start 169 92.7) (end 168.5 93.2) (width 0.15) (layer "F.Cu") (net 16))
 (segment (start 163.2 93.9) (end 163.2 98.5) (width 0.15) (layer "F.Cu") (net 16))
 (segment (start 168.5 93.2) (end 163.9 93.2) (width 0.15) (layer "F.Cu") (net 16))
 (segment (start 169 43.9) (end 169 89.4) (width 0.15) (layer "F.Cu") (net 16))
 (segment (start 163.9 93.2) (end 163.2 93.9) (width 0.15) (layer "F.Cu") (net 16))
 (segment (start 162.7 93.8) (end 163.35 93.15) (width 0.15) (layer "F.Cu") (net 10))
 (segment (start 163.35 93.15) (end 163.35 47.4) (width 0.15) (layer "F.Cu") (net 10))
 (segment (start 162.7 98.5) (end 162.7 93.8) (width 0.15) (layer "F.Cu") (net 10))
 (segment (start 154.7 43.9) (end 154.7 47.4) (width 0.15) (layer "F.Cu") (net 10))
 (via (at 154.7 47.4) (size 0.45) (drill 0.2) (layers "F.Cu" "B.Cu") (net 10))
 (via (at 163.35 47.4) (size 0.45) (drill 0.2) (layers "F.Cu" "B.Cu") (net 10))
 (segment (start 154.7 47.4) (end 163.35 47.4) (width 0.15) (layer "B.Cu") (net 10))
 (segment (start 168 89.4) (end 168 91.2) (width 0.15) (layer "F.Cu") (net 22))
 (segment (start 162.2 98.5) (end 162.2 99.6) (width 0.15) (layer "F.Cu") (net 22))
 (via (at 162.2 99.6) (size 0.45) (drill 0.2) (layers "F.Cu" "B.Cu") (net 22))
 (via (at 168 91.2) (size 0.45) (drill 0.2) (layers "F.Cu" "B.Cu") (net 22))
 (segment (start 168 92.3) (end 162.2 98.1) (width 0.15) (layer "B.Cu") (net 22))
 (segment (start 162.2 98.1) (end 162.2 99.6) (width 0.15) (layer "B.Cu") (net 22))
 (segment (start 168 91.2) (end 168 92.3) (width 0.15) (layer "B.Cu") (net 22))
 (segment (start 154.2 48.2) (end 154.7 48.7) (width 0.15) (layer "F.Cu") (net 5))
 (segment (start 154.7 48.7) (end 154.7 53) (width 0.15) (layer "F.Cu") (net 5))
 (segment (start 154.2 43.9) (end 154.2 48.2) (width 0.15) (layer "F.Cu") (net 5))
 (segment (start 154.7 57.8) (end 154.7 62.1) (width 0.15) (layer "F.Cu") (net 4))
 (segment (start 154.2 53) (end 154.2 57.3) (width 0.15) (layer "F.Cu") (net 4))
 (segment (start 154.2 57.3) (end 154.7 57.8) (width 0.15) (layer "F.Cu") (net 4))
 (segment (start 154.2 62.1) (end 154.2 66.4) (width 0.15) (layer "F.Cu") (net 26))
 (segment (start 154.2 66.4) (end 154.7 66.9) (width 0.15) (layer "F.Cu") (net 26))
 (segment (start 154.7 66.9) (end 154.7 71.2) (width 0.15) (layer "F.Cu") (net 26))
 (segment (start 154.7 76) (end 154.7 80.3) (width 0.15) (layer "F.Cu") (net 25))
 (segment (start 154.2 75.5) (end 154.7 76) (width 0.15) (layer "F.Cu") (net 25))
 (segment (start 154.2 71.2) (end 154.2 75.5) (width 0.15) (layer "F.Cu") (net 25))
 (segment (start 154.7 85.1) (end 154.7 89.4) (width 0.15) (layer "F.Cu") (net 45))
 (segment (start 154.2 80.3) (end 154.2 84.6) (width 0.15) (layer "F.Cu") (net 45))
 (segment (start 154.2 84.6) (end 154.7 85.1) (width 0.15) (layer "F.Cu") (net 45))
 (segment (start 168.5 43.9) (end 168.5 47.95) (width 0.15) (layer "F.Cu") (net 35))
 (segment (start 162.75 92.9) (end 162.75 47.95) (width 0.15) (layer "F.Cu") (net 35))
 (segment (start 154.2 89.4) (end 154.2 92.9) (width 0.15) (layer "F.Cu") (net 35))
 (via (at 168.5 47.95) (size 0.45) (drill 0.2) (layers "F.Cu" "B.Cu") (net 35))
 (via (at 162.75 92.9) (size 0.45) (drill 0.2) (layers "F.Cu" "B.Cu") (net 35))
 (via (at 154.2 92.9) (size 0.45) (drill 0.2) (layers "F.Cu" "B.Cu") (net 35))
 (via (at 162.75 47.95) (size 0.45) (drill 0.2) (layers "F.Cu" "B.Cu") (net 35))
 (segment (start 154.2 92.9) (end 162.75 92.9) (width 0.15) (layer "B.Cu") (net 35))
 (segment (start 168.5 47.95) (end 162.75 47.95) (width 0.15) (layer "B.Cu") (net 35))
 (segment (start 168 80.3) (end 168 84.6) (width 0.15) (layer "F.Cu") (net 14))
 (segment (start 168 84.6) (end 168.5 85.1) (width 0.15) (layer "F.Cu") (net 14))
 (segment (start 168.5 85.1) (end 168.5 89.4) (width 0.15) (layer "F.Cu") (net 14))
 (segment (start 168 75.6) (end 168.5 76.1) (width 0.15) (layer "F.Cu") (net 15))
 (segment (start 168 71.4) (end 168 75.6) (width 0.15) (layer "F.Cu") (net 15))
 (segment (start 168.5 76.1) (end 168.5 80.3) (width 0.15) (layer "F.Cu") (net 15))
 (segment (start 168 62.4) (end 168 66.65) (width 0.15) (layer "F.Cu") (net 29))
 (segment (start 168 66.65) (end 168.5 67.15) (width 0.15) (layer "F.Cu") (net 29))
 (segment (start 168.5 67.15) (end 168.5 71.4) (width 0.15) (layer "F.Cu") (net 29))
 (segment (start 168 57.45) (end 168.5 57.95) (width 0.15) (layer "F.Cu") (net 38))
 (segment (start 168 53) (end 168 57.45) (width 0.15) (layer "F.Cu") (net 38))
 (segment (start 168.5 57.95) (end 168.5 62.4) (width 0.15) (layer "F.Cu") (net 38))
 (segment (start 168 48.2) (end 168.5 48.7) (width 0.15) (layer "F.Cu") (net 34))
 (segment (start 168 43.9) (end 168 48.2) (width 0.15) (layer "F.Cu") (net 34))
 (segment (start 168.5 48.7) (end 168.5 53) (width 0.15) (layer "F.Cu") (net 34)))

